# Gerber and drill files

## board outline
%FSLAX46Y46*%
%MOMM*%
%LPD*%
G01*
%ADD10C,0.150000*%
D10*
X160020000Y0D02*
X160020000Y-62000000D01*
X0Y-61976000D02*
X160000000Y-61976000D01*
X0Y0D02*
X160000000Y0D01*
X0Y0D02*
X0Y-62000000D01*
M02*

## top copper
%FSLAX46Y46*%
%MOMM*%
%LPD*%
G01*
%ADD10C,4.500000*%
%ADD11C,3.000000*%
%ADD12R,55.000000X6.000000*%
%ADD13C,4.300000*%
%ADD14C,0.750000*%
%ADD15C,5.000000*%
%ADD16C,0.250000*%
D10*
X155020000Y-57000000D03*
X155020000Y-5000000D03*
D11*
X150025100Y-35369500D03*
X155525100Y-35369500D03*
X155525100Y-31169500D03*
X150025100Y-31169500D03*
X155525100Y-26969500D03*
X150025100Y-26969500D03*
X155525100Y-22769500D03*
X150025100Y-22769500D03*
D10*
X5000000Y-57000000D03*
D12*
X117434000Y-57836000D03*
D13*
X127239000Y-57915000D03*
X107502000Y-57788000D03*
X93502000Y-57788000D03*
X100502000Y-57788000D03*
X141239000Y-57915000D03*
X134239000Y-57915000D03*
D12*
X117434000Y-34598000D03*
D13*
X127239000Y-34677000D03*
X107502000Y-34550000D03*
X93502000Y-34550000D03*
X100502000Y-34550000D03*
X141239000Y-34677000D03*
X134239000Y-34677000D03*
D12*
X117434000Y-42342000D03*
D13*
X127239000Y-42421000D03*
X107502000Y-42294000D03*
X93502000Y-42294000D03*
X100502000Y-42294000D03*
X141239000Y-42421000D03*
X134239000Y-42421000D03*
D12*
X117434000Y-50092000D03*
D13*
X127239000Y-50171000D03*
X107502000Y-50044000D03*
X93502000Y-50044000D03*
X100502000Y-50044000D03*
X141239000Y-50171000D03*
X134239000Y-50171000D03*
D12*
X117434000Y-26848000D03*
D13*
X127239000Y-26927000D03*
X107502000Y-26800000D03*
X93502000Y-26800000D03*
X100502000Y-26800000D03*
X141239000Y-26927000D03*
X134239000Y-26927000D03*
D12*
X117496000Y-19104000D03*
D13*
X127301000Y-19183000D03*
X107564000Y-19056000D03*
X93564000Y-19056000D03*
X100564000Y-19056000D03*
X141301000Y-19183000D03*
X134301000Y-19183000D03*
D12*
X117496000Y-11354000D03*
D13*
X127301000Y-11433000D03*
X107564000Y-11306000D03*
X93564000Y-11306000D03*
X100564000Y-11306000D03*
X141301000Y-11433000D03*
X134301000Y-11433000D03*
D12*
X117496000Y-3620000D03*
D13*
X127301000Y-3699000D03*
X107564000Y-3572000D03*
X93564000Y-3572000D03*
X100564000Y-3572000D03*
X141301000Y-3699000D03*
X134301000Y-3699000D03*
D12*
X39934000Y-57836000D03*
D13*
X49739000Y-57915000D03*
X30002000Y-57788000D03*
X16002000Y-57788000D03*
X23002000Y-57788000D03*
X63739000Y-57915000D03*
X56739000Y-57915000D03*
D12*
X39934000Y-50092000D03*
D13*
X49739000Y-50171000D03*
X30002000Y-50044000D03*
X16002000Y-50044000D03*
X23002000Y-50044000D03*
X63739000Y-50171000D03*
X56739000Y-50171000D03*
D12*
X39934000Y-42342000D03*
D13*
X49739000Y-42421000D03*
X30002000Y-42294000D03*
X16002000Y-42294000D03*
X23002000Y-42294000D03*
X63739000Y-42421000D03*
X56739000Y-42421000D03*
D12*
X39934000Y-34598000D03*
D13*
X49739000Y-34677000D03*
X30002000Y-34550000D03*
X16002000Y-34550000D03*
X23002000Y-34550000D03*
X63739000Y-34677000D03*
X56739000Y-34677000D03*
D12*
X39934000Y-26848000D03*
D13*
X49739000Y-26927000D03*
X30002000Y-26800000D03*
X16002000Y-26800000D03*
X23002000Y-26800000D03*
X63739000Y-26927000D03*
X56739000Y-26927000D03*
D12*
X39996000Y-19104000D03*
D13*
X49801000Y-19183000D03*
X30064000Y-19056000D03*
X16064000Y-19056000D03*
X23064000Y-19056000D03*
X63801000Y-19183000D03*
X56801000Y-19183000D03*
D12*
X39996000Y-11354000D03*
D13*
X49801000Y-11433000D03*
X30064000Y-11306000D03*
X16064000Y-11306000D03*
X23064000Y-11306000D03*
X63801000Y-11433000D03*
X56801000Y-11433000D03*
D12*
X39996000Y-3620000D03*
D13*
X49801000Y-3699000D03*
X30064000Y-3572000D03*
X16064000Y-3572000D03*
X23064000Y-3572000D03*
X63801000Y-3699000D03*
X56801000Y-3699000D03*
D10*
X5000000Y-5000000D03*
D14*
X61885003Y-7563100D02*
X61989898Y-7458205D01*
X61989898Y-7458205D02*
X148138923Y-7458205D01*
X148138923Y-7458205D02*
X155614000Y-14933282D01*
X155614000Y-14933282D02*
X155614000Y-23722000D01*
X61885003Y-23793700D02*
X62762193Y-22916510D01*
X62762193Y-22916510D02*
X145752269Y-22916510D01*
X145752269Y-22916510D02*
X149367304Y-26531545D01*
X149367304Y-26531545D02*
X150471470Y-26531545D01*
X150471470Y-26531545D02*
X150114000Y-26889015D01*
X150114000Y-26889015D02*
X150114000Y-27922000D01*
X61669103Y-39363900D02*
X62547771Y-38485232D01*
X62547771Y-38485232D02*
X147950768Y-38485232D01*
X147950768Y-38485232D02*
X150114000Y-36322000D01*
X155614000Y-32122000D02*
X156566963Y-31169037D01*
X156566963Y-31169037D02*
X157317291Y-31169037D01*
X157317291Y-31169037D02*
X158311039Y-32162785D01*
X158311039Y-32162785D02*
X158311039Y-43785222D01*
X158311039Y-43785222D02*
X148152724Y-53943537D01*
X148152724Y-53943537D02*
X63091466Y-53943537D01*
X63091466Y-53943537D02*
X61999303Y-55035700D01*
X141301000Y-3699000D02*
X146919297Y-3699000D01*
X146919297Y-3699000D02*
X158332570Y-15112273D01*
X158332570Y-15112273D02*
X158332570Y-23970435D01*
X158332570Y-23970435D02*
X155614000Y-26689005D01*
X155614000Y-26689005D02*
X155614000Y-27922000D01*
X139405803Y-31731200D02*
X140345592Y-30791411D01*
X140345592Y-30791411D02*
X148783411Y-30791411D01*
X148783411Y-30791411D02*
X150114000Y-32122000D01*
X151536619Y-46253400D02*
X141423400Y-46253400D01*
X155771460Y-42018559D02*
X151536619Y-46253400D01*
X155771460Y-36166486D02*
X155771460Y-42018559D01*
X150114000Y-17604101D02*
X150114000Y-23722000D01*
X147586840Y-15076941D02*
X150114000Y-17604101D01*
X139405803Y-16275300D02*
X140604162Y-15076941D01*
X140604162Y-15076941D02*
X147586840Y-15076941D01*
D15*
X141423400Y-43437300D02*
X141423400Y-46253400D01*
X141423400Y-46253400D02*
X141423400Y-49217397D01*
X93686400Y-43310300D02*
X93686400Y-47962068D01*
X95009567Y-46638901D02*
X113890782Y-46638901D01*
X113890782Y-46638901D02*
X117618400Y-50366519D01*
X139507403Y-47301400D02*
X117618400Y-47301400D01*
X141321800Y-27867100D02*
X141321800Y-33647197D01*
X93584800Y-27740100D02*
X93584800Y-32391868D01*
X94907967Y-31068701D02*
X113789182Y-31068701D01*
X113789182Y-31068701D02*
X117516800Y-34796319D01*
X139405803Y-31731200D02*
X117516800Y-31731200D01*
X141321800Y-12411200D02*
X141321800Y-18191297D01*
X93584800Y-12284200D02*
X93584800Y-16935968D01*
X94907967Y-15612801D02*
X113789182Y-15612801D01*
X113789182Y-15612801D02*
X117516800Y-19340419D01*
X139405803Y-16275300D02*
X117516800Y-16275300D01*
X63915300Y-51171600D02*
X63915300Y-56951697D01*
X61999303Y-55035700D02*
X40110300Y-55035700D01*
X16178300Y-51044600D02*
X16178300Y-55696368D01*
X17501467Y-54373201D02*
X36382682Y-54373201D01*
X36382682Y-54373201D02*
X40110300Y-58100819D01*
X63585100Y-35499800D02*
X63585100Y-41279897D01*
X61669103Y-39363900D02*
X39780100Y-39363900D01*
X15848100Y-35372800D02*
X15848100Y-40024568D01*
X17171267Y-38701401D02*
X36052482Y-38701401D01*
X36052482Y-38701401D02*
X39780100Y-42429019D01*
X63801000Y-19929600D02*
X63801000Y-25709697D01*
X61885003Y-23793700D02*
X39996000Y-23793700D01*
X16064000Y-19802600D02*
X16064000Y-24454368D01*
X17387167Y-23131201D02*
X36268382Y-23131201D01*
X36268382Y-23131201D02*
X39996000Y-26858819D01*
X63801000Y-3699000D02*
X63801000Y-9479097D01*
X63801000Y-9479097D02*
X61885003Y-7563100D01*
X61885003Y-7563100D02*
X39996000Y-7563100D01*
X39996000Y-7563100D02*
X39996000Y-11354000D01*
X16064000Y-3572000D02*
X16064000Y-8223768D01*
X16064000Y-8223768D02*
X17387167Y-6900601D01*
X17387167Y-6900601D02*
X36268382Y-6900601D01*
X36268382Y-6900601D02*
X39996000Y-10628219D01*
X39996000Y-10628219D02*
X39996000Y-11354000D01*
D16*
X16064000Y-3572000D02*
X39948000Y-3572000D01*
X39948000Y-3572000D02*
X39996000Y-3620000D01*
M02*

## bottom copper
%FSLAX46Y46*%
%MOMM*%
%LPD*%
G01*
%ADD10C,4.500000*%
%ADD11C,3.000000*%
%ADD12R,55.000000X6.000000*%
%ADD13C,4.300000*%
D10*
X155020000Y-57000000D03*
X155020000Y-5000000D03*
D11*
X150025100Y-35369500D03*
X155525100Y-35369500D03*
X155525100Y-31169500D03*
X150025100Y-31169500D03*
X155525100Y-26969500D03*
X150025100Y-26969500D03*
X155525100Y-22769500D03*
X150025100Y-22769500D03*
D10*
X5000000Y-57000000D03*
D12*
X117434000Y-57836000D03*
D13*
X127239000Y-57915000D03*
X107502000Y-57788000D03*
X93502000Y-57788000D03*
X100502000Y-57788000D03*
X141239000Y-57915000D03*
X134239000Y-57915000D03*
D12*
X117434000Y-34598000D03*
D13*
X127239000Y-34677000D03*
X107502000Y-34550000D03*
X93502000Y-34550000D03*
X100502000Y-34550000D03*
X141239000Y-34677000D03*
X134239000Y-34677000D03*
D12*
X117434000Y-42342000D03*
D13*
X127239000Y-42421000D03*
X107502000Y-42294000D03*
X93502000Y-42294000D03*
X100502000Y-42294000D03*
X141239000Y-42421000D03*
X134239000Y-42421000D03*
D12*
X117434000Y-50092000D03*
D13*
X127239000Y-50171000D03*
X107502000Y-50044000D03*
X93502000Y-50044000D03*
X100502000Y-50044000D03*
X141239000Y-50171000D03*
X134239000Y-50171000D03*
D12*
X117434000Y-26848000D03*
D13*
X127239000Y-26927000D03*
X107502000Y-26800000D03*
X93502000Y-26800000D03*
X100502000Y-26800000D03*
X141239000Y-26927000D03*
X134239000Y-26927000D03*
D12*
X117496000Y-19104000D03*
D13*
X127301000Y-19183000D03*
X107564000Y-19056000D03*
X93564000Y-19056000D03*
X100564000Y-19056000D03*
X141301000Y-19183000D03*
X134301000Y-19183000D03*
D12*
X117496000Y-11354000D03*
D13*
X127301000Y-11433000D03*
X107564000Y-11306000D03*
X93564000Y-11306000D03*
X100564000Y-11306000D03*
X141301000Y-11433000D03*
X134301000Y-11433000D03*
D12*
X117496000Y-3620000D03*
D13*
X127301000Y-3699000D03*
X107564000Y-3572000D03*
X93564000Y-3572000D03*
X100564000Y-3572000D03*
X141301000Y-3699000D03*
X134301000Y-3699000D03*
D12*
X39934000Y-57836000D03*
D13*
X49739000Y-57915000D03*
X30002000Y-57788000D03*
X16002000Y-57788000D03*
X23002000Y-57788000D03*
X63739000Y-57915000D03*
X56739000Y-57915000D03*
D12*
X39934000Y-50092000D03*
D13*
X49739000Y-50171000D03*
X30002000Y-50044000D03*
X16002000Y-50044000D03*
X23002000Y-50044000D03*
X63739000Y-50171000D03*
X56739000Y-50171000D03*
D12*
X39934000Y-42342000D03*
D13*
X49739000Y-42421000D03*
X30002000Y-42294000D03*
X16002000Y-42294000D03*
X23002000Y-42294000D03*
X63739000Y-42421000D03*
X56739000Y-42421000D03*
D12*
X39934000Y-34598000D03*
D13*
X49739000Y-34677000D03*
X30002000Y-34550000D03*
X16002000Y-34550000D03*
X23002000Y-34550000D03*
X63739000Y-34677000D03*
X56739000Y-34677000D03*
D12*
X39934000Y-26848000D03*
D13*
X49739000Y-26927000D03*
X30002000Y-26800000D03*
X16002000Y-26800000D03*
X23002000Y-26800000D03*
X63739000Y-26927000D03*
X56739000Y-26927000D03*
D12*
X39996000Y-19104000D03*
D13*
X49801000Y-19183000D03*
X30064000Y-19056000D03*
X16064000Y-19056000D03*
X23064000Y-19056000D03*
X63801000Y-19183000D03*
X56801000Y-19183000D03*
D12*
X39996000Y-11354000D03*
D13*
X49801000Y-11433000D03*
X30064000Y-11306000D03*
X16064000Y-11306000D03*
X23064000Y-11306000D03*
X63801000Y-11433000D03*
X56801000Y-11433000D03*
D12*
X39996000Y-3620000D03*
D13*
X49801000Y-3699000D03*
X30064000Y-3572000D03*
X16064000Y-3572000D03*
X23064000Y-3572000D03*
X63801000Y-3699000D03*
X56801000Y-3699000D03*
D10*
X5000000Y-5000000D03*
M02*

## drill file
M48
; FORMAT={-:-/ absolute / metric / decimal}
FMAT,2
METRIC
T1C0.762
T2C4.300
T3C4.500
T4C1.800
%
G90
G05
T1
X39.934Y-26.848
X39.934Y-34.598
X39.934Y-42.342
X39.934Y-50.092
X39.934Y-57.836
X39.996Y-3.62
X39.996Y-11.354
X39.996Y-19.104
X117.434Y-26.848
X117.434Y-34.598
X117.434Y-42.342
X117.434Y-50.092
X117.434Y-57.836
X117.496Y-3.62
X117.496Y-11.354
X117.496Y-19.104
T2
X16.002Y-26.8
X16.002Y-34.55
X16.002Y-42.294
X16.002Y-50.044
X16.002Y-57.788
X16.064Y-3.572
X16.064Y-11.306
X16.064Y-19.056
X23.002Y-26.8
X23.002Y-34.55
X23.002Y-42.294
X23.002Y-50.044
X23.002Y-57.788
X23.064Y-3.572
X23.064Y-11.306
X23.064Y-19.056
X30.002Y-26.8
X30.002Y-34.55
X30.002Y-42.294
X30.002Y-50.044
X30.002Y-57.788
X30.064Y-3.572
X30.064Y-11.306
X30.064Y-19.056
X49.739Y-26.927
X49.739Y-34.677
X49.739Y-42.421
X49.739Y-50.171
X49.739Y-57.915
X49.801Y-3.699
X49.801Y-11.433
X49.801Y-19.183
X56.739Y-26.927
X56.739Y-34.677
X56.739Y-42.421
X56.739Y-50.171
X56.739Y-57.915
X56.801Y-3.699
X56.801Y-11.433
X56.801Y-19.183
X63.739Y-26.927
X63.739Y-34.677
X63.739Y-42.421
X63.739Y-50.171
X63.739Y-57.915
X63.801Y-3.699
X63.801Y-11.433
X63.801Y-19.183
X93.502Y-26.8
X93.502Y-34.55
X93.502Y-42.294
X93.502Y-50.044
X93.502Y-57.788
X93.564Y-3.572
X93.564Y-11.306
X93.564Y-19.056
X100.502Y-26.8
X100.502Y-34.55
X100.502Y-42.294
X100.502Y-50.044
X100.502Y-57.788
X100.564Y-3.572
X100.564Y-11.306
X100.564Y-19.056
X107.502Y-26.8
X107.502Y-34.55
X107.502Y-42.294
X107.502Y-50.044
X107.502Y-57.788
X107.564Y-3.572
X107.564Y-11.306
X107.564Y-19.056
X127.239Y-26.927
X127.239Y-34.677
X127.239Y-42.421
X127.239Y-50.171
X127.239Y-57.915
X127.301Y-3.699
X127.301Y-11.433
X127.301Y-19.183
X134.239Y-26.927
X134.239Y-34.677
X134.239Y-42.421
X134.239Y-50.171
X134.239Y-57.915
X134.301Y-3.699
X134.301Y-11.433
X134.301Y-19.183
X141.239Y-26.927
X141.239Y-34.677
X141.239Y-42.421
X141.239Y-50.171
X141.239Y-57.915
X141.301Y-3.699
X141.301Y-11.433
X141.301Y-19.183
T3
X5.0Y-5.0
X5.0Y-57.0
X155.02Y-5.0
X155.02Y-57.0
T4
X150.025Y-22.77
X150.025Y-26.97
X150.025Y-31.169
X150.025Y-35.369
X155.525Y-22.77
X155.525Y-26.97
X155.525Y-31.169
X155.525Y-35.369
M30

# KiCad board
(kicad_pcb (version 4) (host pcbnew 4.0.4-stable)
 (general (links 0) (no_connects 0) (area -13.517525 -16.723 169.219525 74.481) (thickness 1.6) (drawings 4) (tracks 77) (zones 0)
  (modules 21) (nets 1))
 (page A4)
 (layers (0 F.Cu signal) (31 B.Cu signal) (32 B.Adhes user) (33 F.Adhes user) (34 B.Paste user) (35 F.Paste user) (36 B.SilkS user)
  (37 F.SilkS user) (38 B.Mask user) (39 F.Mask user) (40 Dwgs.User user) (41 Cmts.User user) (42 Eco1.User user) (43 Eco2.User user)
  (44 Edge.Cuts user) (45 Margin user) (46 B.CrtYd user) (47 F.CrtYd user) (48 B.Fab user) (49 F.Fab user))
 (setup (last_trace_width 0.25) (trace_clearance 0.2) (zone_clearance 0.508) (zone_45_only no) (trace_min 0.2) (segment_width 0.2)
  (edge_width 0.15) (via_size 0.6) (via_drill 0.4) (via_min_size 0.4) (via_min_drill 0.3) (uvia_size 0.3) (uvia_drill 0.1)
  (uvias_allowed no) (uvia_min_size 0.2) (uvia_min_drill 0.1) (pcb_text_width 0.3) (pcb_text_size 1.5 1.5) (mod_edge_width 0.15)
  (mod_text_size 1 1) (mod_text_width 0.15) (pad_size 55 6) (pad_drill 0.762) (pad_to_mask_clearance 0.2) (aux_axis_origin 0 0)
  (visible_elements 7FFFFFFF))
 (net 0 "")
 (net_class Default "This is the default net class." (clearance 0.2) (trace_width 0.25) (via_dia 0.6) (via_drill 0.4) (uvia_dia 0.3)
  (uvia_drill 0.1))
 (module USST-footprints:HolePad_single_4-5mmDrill (layer F.Cu) (at 154.258 49.634)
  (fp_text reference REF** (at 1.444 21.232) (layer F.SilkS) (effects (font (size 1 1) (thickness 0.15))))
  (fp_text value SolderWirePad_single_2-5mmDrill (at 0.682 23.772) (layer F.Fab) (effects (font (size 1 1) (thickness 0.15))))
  (pad "" thru_hole circle (at 0.762 7.366) (size 4.5 4.5) (drill 4.5) (layers *.Cu *.Mask)))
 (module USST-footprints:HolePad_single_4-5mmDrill (layer F.Cu) (at 154.258 -2.366)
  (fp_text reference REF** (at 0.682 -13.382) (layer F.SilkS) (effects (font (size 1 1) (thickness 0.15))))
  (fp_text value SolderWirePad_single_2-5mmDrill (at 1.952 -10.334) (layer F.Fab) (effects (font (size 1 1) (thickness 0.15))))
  (pad "" thru_hole circle (at 0.762 7.366) (size 4.5 4.5) (drill 4.5) (layers *.Cu *.Mask)))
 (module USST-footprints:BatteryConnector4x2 (layer F.Cu) (at 150.0251 35.3695)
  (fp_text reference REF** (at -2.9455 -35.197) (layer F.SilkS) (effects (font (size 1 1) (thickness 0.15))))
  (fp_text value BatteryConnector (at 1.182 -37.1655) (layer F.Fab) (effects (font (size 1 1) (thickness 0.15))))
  (pad "" np_thru_hole circle (at 0 0) (size 3 3) (drill 1.8) (layers *.Cu))
  (pad "" np_thru_hole circle (at 5.5 0) (size 3 3) (drill 1.8) (layers *.Cu))
  (pad "" np_thru_hole circle (at 5.5 -4.2) (size 3 3) (drill 1.8) (layers *.Cu))
  (pad "" np_thru_hole circle (at 0 -4.2) (size 3 3) (drill 1.8) (layers *.Cu))
  (pad "" np_thru_hole circle (at 5.5 -8.4) (size 3 3) (drill 1.8) (layers *.Cu))
  (pad "" np_thru_hole circle (at 0 -8.4) (size 3 3) (drill 1.8) (layers *.Cu))
  (pad "" np_thru_hole circle (at 5.5 -12.6) (size 3 3) (drill 1.8) (layers *.Cu))
  (pad "" np_thru_hole circle (at 0 -12.6) (size 3 3) (drill 1.8) (layers *.Cu)))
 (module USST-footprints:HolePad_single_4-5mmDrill (layer F.Cu) (at 4.238 49.634)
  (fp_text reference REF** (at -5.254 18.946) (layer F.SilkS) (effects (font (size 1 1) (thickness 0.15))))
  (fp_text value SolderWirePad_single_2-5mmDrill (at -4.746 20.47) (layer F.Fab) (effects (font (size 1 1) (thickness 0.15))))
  (pad "" thru_hole circle (at 0.762 7.366) (size 4.5 4.5) (drill 4.5) (layers *.Cu *.Mask)))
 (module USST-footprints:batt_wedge (layer F.Cu) (at 117.434 57.836)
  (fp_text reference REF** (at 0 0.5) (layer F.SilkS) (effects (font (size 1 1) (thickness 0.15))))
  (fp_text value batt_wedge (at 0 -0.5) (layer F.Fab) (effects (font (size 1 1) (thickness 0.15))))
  (pad 8 thru_hole rect (at 0 0) (size 55 6) (drill 0.762) (layers F.Cu F.Paste))
  (pad "" thru_hole circle (at 9.805 0.079) (size 4.3 4.3) (drill 4.3) (layers *.Cu *.Mask))
  (pad "" thru_hole circle (at -9.932 -0.048) (size 4.3 4.3) (drill 4.3) (layers *.Cu *.Mask))
  (pad "" thru_hole circle (at -23.932 -0.048) (size 4.3 4.3) (drill 4.3) (layers *.Cu *.Mask))
  (pad "" thru_hole circle (at -16.932 -0.048) (size 4.3 4.3) (drill 4.3) (layers *.Cu *.Mask))
  (pad "" thru_hole circle (at 23.805 0.079) (size 4.3 4.3) (drill 4.3) (layers *.Cu *.Mask))
  (pad "" thru_hole circle (at 16.805 0.079) (size 4.3 4.3) (drill 4.3) (layers *.Cu *.Mask)))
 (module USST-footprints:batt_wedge (layer F.Cu) (at 117.434 34.598)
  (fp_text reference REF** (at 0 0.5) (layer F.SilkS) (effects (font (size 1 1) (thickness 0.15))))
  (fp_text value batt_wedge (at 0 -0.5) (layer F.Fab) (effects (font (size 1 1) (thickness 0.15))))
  (pad 5 thru_hole rect (at 0 0) (size 55 6) (drill 0.762) (layers F.Cu F.Paste))
  (pad "" thru_hole circle (at 9.805 0.079) (size 4.3 4.3) (drill 4.3) (layers *.Cu *.Mask))
  (pad "" thru_hole circle (at -9.932 -0.048) (size 4.3 4.3) (drill 4.3) (layers *.Cu *.Mask))
  (pad "" thru_hole circle (at -23.932 -0.048) (size 4.3 4.3) (drill 4.3) (layers *.Cu *.Mask))
  (pad "" thru_hole circle (at -16.932 -0.048) (size 4.3 4.3) (drill 4.3) (layers *.Cu *.Mask))
  (pad "" thru_hole circle (at 23.805 0.079) (size 4.3 4.3) (drill 4.3) (layers *.Cu *.Mask))
  (pad "" thru_hole circle (at 16.805 0.079) (size 4.3 4.3) (drill 4.3) (layers *.Cu *.Mask)))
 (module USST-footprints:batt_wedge (layer F.Cu) (at 117.434 42.342)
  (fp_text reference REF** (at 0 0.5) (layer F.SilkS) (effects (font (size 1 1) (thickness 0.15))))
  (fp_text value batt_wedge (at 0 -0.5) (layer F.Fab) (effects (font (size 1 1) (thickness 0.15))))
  (pad 6 thru_hole rect (at 0 0) (size 55 6) (drill 0.762) (layers F.Cu F.Paste))
  (pad "" thru_hole circle (at 9.805 0.079) (size 4.3 4.3) (drill 4.3) (layers *.Cu *.Mask))
  (pad "" thru_hole circle (at -9.932 -0.048) (size 4.3 4.3) (drill 4.3) (layers *.Cu *.Mask))
  (pad "" thru_hole circle (at -23.932 -0.048) (size 4.3 4.3) (drill 4.3) (layers *.Cu *.Mask))
  (pad "" thru_hole circle (at -16.932 -0.048) (size 4.3 4.3) (drill 4.3) (layers *.Cu *.Mask))
  (pad "" thru_hole circle (at 23.805 0.079) (size 4.3 4.3) (drill 4.3) (layers *.Cu *.Mask))
  (pad "" thru_hole circle (at 16.805 0.079) (size 4.3 4.3) (drill 4.3) (layers *.Cu *.Mask)))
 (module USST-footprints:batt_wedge (layer F.Cu) (at 117.434 50.092)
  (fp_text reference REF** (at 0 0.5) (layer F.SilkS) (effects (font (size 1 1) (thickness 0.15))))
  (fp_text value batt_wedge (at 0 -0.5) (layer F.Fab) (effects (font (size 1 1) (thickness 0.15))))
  (pad 7 thru_hole rect (at 0 0) (size 55 6) (drill 0.762) (layers F.Cu F.Paste))
  (pad "" thru_hole circle (at 9.805 0.079) (size 4.3 4.3) (drill 4.3) (layers *.Cu *.Mask))
  (pad "" thru_hole circle (at -9.932 -0.048) (size 4.3 4.3) (drill 4.3) (layers *.Cu *.Mask))
  (pad "" thru_hole circle (at -23.932 -0.048) (size 4.3 4.3) (drill 4.3) (layers *.Cu *.Mask))
  (pad "" thru_hole circle (at -16.932 -0.048) (size 4.3 4.3) (drill 4.3) (layers *.Cu *.Mask))
  (pad "" thru_hole circle (at 23.805 0.079) (size 4.3 4.3) (drill 4.3) (layers *.Cu *.Mask))
  (pad "" thru_hole circle (at 16.805 0.079) (size 4.3 4.3) (drill 4.3) (layers *.Cu *.Mask)))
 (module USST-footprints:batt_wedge (layer F.Cu) (at 117.434 26.848)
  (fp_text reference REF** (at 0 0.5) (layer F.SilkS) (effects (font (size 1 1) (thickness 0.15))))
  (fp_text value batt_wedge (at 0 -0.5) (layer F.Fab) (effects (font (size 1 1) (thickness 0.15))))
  (pad 4 thru_hole rect (at 0 0) (size 55 6) (drill 0.762) (layers F.Cu F.Paste))
  (pad "" thru_hole circle (at 9.805 0.079) (size 4.3 4.3) (drill 4.3) (layers *.Cu *.Mask))
  (pad "" thru_hole circle (at -9.932 -0.048) (size 4.3 4.3) (drill 4.3) (layers *.Cu *.Mask))
  (pad "" thru_hole circle (at -23.932 -0.048) (size 4.3 4.3) (drill 4.3) (layers *.Cu *.Mask))
  (pad "" thru_hole circle (at -16.932 -0.048) (size 4.3 4.3) (drill 4.3) (layers *.Cu *.Mask))
  (pad "" thru_hole circle (at 23.805 0.079) (size 4.3 4.3) (drill 4.3) (layers *.Cu *.Mask))
  (pad "" thru_hole circle (at 16.805 0.079) (size 4.3 4.3) (drill 4.3) (layers *.Cu *.Mask)))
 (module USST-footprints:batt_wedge (layer F.Cu) (at 117.496 19.104)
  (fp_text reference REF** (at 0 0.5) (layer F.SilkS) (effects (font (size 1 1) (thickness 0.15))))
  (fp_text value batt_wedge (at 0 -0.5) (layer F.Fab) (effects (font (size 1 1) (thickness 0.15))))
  (pad 3 thru_hole rect (at 0 0) (size 55 6) (drill 0.762) (layers F.Cu F.Paste))
  (pad "" thru_hole circle (at 9.805 0.079) (size 4.3 4.3) (drill 4.3) (layers *.Cu *.Mask))
  (pad "" thru_hole circle (at -9.932 -0.048) (size 4.3 4.3) (drill 4.3) (layers *.Cu *.Mask))
  (pad "" thru_hole circle (at -23.932 -0.048) (size 4.3 4.3) (drill 4.3) (layers *.Cu *.Mask))
  (pad "" thru_hole circle (at -16.932 -0.048) (size 4.3 4.3) (drill 4.3) (layers *.Cu *.Mask))
  (pad "" thru_hole circle (at 23.805 0.079) (size 4.3 4.3) (drill 4.3) (layers *.Cu *.Mask))
  (pad "" thru_hole circle (at 16.805 0.079) (size 4.3 4.3) (drill 4.3) (layers *.Cu *.Mask)))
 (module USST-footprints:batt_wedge (layer F.Cu) (at 117.496 11.354)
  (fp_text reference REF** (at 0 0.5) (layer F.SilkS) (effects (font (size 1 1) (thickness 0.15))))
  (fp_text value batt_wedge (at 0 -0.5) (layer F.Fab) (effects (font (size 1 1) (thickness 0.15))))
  (pad 2 thru_hole rect (at 0 0) (size 55 6) (drill 0.762) (layers F.Cu F.Paste))
  (pad "" thru_hole circle (at 9.805 0.079) (size 4.3 4.3) (drill 4.3) (layers *.Cu *.Mask))
  (pad "" thru_hole circle (at -9.932 -0.048) (size 4.3 4.3) (drill 4.3) (layers *.Cu *.Mask))
  (pad "" thru_hole circle (at -23.932 -0.048) (size 4.3 4.3) (drill 4.3) (layers *.Cu *.Mask))
  (pad "" thru_hole circle (at -16.932 -0.048) (size 4.3 4.3) (drill 4.3) (layers *.Cu *.Mask))
  (pad "" thru_hole circle (at 23.805 0.079) (size 4.3 4.3) (drill 4.3) (layers *.Cu *.Mask))
  (pad "" thru_hole circle (at 16.805 0.079) (size 4.3 4.3) (drill 4.3) (layers *.Cu *.Mask)))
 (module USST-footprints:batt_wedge (layer F.Cu) (at 117.496 3.62)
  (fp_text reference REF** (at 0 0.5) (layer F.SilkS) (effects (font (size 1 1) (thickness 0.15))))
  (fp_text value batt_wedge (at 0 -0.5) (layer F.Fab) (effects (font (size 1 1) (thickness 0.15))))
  (pad 1 thru_hole rect (at 0 0) (size 55 6) (drill 0.762) (layers F.Cu F.Paste))
  (pad "" thru_hole circle (at 9.805 0.079) (size 4.3 4.3) (drill 4.3) (layers *.Cu *.Mask))
  (pad "" thru_hole circle (at -9.932 -0.048) (size 4.3 4.3) (drill 4.3) (layers *.Cu *.Mask))
  (pad "" thru_hole circle (at -23.932 -0.048) (size 4.3 4.3) (drill 4.3) (layers *.Cu *.Mask))
  (pad "" thru_hole circle (at -16.932 -0.048) (size 4.3 4.3) (drill 4.3) (layers *.Cu *.Mask))
  (pad "" thru_hole circle (at 23.805 0.079) (size 4.3 4.3) (drill 4.3) (layers *.Cu *.Mask))
  (pad "" thru_hole circle (at 16.805 0.079) (size 4.3 4.3) (drill 4.3) (layers *.Cu *.Mask)))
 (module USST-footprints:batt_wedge (layer F.Cu) (at 39.934 57.836)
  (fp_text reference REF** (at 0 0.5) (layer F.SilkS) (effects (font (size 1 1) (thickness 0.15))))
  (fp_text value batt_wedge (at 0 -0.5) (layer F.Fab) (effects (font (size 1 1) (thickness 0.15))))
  (pad 8 thru_hole rect (at 0 0) (size 55 6) (drill 0.762) (layers F.Cu F.Paste))
  (pad "" thru_hole circle (at 9.805 0.079) (size 4.3 4.3) (drill 4.3) (layers *.Cu *.Mask))
  (pad "" thru_hole circle (at -9.932 -0.048) (size 4.3 4.3) (drill 4.3) (layers *.Cu *.Mask))
  (pad "" thru_hole circle (at -23.932 -0.048) (size 4.3 4.3) (drill 4.3) (layers *.Cu *.Mask))
  (pad "" thru_hole circle (at -16.932 -0.048) (size 4.3 4.3) (drill 4.3) (layers *.Cu *.Mask))
  (pad "" thru_hole circle (at 23.805 0.079) (size 4.3 4.3) (drill 4.3) (layers *.Cu *.Mask))
  (pad "" thru_hole circle (at 16.805 0.079) (size 4.3 4.3) (drill 4.3) (layers *.Cu *.Mask)))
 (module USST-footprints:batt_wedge (layer F.Cu) (at 39.934 50.092)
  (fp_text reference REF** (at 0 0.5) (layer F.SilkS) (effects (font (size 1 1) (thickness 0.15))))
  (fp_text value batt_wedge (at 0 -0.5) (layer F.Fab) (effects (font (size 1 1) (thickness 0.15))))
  (pad 7 thru_hole rect (at 0 0) (size 55 6) (drill 0.762) (layers F.Cu F.Paste))
  (pad "" thru_hole circle (at 9.805 0.079) (size 4.3 4.3) (drill 4.3) (layers *.Cu *.Mask))
  (pad "" thru_hole circle (at -9.932 -0.048) (size 4.3 4.3) (drill 4.3) (layers *.Cu *.Mask))
  (pad "" thru_hole circle (at -23.932 -0.048) (size 4.3 4.3) (drill 4.3) (layers *.Cu *.Mask))
  (pad "" thru_hole circle (at -16.932 -0.048) (size 4.3 4.3) (drill 4.3) (layers *.Cu *.Mask))
  (pad "" thru_hole circle (at 23.805 0.079) (size 4.3 4.3) (drill 4.3) (layers *.Cu *.Mask))
  (pad "" thru_hole circle (at 16.805 0.079) (size 4.3 4.3) (drill 4.3) (layers *.Cu *.Mask)))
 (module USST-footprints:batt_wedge (layer F.Cu) (at 39.934 42.342)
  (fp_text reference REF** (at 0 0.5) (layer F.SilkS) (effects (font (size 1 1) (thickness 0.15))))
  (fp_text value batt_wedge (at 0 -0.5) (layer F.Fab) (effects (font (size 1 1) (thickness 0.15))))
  (pad 6 thru_hole rect (at 0 0) (size 55 6) (drill 0.762) (layers F.Cu F.Paste))
  (pad "" thru_hole circle (at 9.805 0.079) (size 4.3 4.3) (drill 4.3) (layers *.Cu *.Mask))
  (pad "" thru_hole circle (at -9.932 -0.048) (size 4.3 4.3) (drill 4.3) (layers *.Cu *.Mask))
  (pad "" thru_hole circle (at -23.932 -0.048) (size 4.3 4.3) (drill 4.3) (layers *.Cu *.Mask))
  (pad "" thru_hole circle (at -16.932 -0.048) (size 4.3 4.3) (drill 4.3) (layers *.Cu *.Mask))
  (pad "" thru_hole circle (at 23.805 0.079) (size 4.3 4.3) (drill 4.3) (layers *.Cu *.Mask))
  (pad "" thru_hole circle (at 16.805 0.079) (size 4.3 4.3) (drill 4.3) (layers *.Cu *.Mask)))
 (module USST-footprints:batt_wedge (layer F.Cu) (at 39.934 34.598)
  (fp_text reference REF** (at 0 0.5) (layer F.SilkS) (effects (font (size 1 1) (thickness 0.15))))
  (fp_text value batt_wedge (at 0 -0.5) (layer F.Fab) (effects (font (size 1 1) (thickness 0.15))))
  (pad 5 thru_hole rect (at 0 0) (size 55 6) (drill 0.762) (layers F.Cu F.Paste))
  (pad "" thru_hole circle (at 9.805 0.079) (size 4.3 4.3) (drill 4.3) (layers *.Cu *.Mask))
  (pad "" thru_hole circle (at -9.932 -0.048) (size 4.3 4.3) (drill 4.3) (layers *.Cu *.Mask))
  (pad "" thru_hole circle (at -23.932 -0.048) (size 4.3 4.3) (drill 4.3) (layers *.Cu *.Mask))
  (pad "" thru_hole circle (at -16.932 -0.048) (size 4.3 4.3) (drill 4.3) (layers *.Cu *.Mask))
  (pad "" thru_hole circle (at 23.805 0.079) (size 4.3 4.3) (drill 4.3) (layers *.Cu *.Mask))
  (pad "" thru_hole circle (at 16.805 0.079) (size 4.3 4.3) (drill 4.3) (layers *.Cu *.Mask)))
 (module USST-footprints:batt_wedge (layer F.Cu) (at 39.934 26.848)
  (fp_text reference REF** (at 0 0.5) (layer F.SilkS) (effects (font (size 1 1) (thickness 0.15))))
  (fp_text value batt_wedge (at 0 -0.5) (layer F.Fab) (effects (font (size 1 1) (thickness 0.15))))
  (pad 4 thru_hole rect (at 0 0) (size 55 6) (drill 0.762) (layers F.Cu F.Paste))
  (pad "" thru_hole circle (at 9.805 0.079) (size 4.3 4.3) (drill 4.3) (layers *.Cu *.Mask))
  (pad "" thru_hole circle (at -9.932 -0.048) (size 4.3 4.3) (drill 4.3) (layers *.Cu *.Mask))
  (pad "" thru_hole circle (at -23.932 -0.048) (size 4.3 4.3) (drill 4.3) (layers *.Cu *.Mask))
  (pad "" thru_hole circle (at -16.932 -0.048) (size 4.3 4.3) (drill 4.3) (layers *.Cu *.Mask))
  (pad "" thru_hole circle (at 23.805 0.079) (size 4.3 4.3) (drill 4.3) (layers *.Cu *.Mask))
  (pad "" thru_hole circle (at 16.805 0.079) (size 4.3 4.3) (drill 4.3) (layers *.Cu *.Mask)))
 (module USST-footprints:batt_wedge (layer F.Cu) (at 39.996 19.104)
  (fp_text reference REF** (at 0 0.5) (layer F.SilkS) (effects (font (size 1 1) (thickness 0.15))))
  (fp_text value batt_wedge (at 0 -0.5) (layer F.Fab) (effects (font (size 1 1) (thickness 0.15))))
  (pad 3 thru_hole rect (at 0 0) (size 55 6) (drill 0.762) (layers F.Cu F.Paste))
  (pad "" thru_hole circle (at 9.805 0.079) (size 4.3 4.3) (drill 4.3) (layers *.Cu *.Mask))
  (pad "" thru_hole circle (at -9.932 -0.048) (size 4.3 4.3) (drill 4.3) (layers *.Cu *.Mask))
  (pad "" thru_hole circle (at -23.932 -0.048) (size 4.3 4.3) (drill 4.3) (layers *.Cu *.Mask))
  (pad "" thru_hole circle (at -16.932 -0.048) (size 4.3 4.3) (drill 4.3) (layers *.Cu *.Mask))
  (pad "" thru_hole circle (at 23.805 0.079) (size 4.3 4.3) (drill 4.3) (layers *.Cu *.Mask))
  (pad "" thru_hole circle (at 16.805 0.079) (size 4.3 4.3) (drill 4.3) (layers *.Cu *.Mask)))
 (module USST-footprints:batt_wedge (layer F.Cu) (at 39.996 11.354)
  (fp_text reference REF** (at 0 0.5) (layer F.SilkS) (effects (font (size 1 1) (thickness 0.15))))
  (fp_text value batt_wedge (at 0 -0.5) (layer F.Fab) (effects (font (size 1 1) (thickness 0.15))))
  (pad 2 thru_hole rect (at 0 0) (size 55 6) (drill 0.762) (layers F.Cu F.Paste))
  (pad "" thru_hole circle (at 9.805 0.079) (size 4.3 4.3) (drill 4.3) (layers *.Cu *.Mask))
  (pad "" thru_hole circle (at -9.932 -0.048) (size 4.3 4.3) (drill 4.3) (layers *.Cu *.Mask))
  (pad "" thru_hole circle (at -23.932 -0.048) (size 4.3 4.3) (drill 4.3) (layers *.Cu *.Mask))
  (pad "" thru_hole circle (at -16.932 -0.048) (size 4.3 4.3) (drill 4.3) (layers *.Cu *.Mask))
  (pad "" thru_hole circle (at 23.805 0.079) (size 4.3 4.3) (drill 4.3) (layers *.Cu *.Mask))
  (pad "" thru_hole circle (at 16.805 0.079) (size 4.3 4.3) (drill 4.3) (layers *.Cu *.Mask)))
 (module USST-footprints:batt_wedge (layer F.Cu) (at 39.996 3.62)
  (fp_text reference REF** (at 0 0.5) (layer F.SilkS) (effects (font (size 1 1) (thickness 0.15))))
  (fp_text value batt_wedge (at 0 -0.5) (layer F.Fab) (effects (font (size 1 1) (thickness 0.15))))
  (pad 1 thru_hole rect (at 0 0) (size 55 6) (drill 0.762) (layers F.Cu F.Paste))
  (pad "" thru_hole circle (at 9.805 0.079) (size 4.3 4.3) (drill 4.3) (layers *.Cu *.Mask))
  (pad "" thru_hole circle (at -9.932 -0.048) (size 4.3 4.3) (drill 4.3) (layers *.Cu *.Mask))
  (pad "" thru_hole circle (at -23.932 -0.048) (size 4.3 4.3) (drill 4.3) (layers *.Cu *.Mask))
  (pad "" thru_hole circle (at -16.932 -0.048) (size 4.3 4.3) (drill 4.3) (layers *.Cu *.Mask))
  (pad "" thru_hole circle (at 23.805 0.079) (size 4.3 4.3) (drill 4.3) (layers *.Cu *.Mask))
  (pad "" thru_hole circle (at 16.805 0.079) (size 4.3 4.3) (drill 4.3) (layers *.Cu *.Mask)))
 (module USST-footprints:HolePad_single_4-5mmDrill (layer F.Cu) (at 4.238 -2.366)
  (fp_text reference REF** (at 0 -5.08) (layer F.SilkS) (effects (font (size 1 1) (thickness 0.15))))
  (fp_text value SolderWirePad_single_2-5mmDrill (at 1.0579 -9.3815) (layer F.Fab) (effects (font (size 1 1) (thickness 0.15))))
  (pad "" thru_hole circle (at 0.762 7.366) (size 4.5 4.5) (drill 4.5) (layers *.Cu *.Mask)))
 (gr_line (start 160.02 0) (end 160.02 62) (layer Edge.Cuts) (width 0.15))
 (gr_line (start 0 61.976) (end 160 61.976) (layer Edge.Cuts) (width 0.15))
 (gr_line (start 0 0) (end 160 0) (layer Edge.Cuts) (width 0.15))
 (gr_line (start 0 0) (end 0 62) (layer Edge.Cuts) (width 0.15))
 (segment (start 61.885003 7.5631) (end 61.989898 7.458205) (width 0.75) (layer F.Cu) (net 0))
 (segment (start 61.989898 7.458205) (end 148.138923 7.458205) (width 0.75) (layer F.Cu) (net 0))
 (segment (start 148.138923 7.458205) (end 155.614 14.933282) (width 0.75) (layer F.Cu) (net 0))
 (segment (start 155.614 14.933282) (end 155.614 23.722) (width 0.75) (layer F.Cu) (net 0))
 (segment (start 61.885003 23.7937) (end 62.762193 22.91651) (width 0.75) (layer F.Cu) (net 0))
 (segment (start 62.762193 22.91651) (end 145.752269 22.91651) (width 0.75) (layer F.Cu) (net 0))
 (segment (start 145.752269 22.91651) (end 149.367304 26.531545) (width 0.75) (layer F.Cu) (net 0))
 (segment (start 149.367304 26.531545) (end 150.47147 26.531545) (width 0.75) (layer F.Cu) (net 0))
 (segment (start 150.47147 26.531545) (end 150.114 26.889015) (width 0.75) (layer F.Cu) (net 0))
 (segment (start 150.114 26.889015) (end 150.114 27.922) (width 0.75) (layer F.Cu) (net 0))
 (segment (start 61.669103 39.3639) (end 62.547771 38.485232) (width 0.75) (layer F.Cu) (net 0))
 (segment (start 62.547771 38.485232) (end 147.950768 38.485232) (width 0.75) (layer F.Cu) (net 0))
 (segment (start 147.950768 38.485232) (end 150.114 36.322) (width 0.75) (layer F.Cu) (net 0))
 (segment (start 155.614 32.122) (end 156.566963 31.169037) (width 0.75) (layer F.Cu) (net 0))
 (segment (start 156.566963 31.169037) (end 157.317291 31.169037) (width 0.75) (layer F.Cu) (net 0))
 (segment (start 157.317291 31.169037) (end 158.311039 32.162785) (width 0.75) (layer F.Cu) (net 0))
 (segment (start 158.311039 32.162785) (end 158.311039 43.785222) (width 0.75) (layer F.Cu) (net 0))
 (segment (start 158.311039 43.785222) (end 148.152724 53.943537) (width 0.75) (layer F.Cu) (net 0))
 (segment (start 148.152724 53.943537) (end 63.091466 53.943537) (width 0.75) (layer F.Cu) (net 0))
 (segment (start 63.091466 53.943537) (end 61.999303 55.0357) (width 0.75) (layer F.Cu) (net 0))
 (segment (start 141.301 3.699) (end 146.919297 3.699) (width 0.75) (layer F.Cu) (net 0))
 (segment (start 146.919297 3.699) (end 158.33257 15.112273) (width 0.75) (layer F.Cu) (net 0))
 (segment (start 158.33257 15.112273) (end 158.33257 23.970435) (width 0.75) (layer F.Cu) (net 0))
 (segment (start 158.33257 23.970435) (end 155.614 26.689005) (width 0.75) (layer F.Cu) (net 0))
 (segment (start 155.614 26.689005) (end 155.614 27.922) (width 0.75) (layer F.Cu) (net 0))
 (segment (start 139.405803 31.7312) (end 140.345592 30.791411) (width 0.75) (layer F.Cu) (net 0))
 (segment (start 140.345592 30.791411) (end 148.783411 30.791411) (width 0.75) (layer F.Cu) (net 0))
 (segment (start 148.783411 30.791411) (end 150.114 32.122) (width 0.75) (layer F.Cu) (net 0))
 (segment (start 151.536619 46.2534) (end 141.4234 46.2534) (width 0.75) (layer F.Cu) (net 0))
 (segment (start 155.77146 42.018559) (end 151.536619 46.2534) (width 0.75) (layer F.Cu) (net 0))
 (segment (start 155.77146 36.166486) (end 155.77146 42.018559) (width 0.75) (layer F.Cu) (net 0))
 (segment (start 150.114 17.604101) (end 150.114 23.722) (width 0.75) (layer F.Cu) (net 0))
 (segment (start 147.58684 15.076941) (end 150.114 17.604101) (width 0.75) (layer F.Cu) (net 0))
 (segment (start 139.405803 16.2753) (end 140.604162 15.076941) (width 0.75) (layer F.Cu) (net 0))
 (segment (start 140.604162 15.076941) (end 147.58684 15.076941) (width 0.75) (layer F.Cu) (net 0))
 (segment (start 141.4234 43.4373) (end 141.4234 46.2534) (width 5) (layer F.Cu) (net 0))
 (segment (start 141.4234 46.2534) (end 141.4234 49.217397) (width 5) (layer F.Cu) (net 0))
 (segment (start 93.6864 43.3103) (end 93.6864 47.962068) (width 5) (layer F.Cu) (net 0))
 (segment (start 95.009567 46.638901) (end 113.890782 46.638901) (width 5) (layer F.Cu) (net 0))
 (segment (start 113.890782 46.638901) (end 117.6184 50.366519) (width 5) (layer F.Cu) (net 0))
 (segment (start 139.507403 47.3014) (end 117.6184 47.3014) (width 5) (layer F.Cu) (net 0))
 (segment (start 141.3218 27.8671) (end 141.3218 33.647197) (width 5) (layer F.Cu) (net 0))
 (segment (start 93.5848 27.7401) (end 93.5848 32.391868) (width 5) (layer F.Cu) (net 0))
 (segment (start 94.907967 31.068701) (end 113.789182 31.068701) (width 5) (layer F.Cu) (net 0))
 (segment (start 113.789182 31.068701) (end 117.5168 34.796319) (width 5) (layer F.Cu) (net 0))
 (segment (start 139.405803 31.7312) (end 117.5168 31.7312) (width 5) (layer F.Cu) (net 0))
 (segment (start 141.3218 12.4112) (end 141.3218 18.191297) (width 5) (layer F.Cu) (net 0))
 (segment (start 93.5848 12.2842) (end 93.5848 16.935968) (width 5) (layer F.Cu) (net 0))
 (segment (start 94.907967 15.612801) (end 113.789182 15.612801) (width 5) (layer F.Cu) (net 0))
 (segment (start 113.789182 15.612801) (end 117.5168 19.340419) (width 5) (layer F.Cu) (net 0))
 (segment (start 139.405803 16.2753) (end 117.5168 16.2753) (width 5) (layer F.Cu) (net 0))
 (segment (start 63.9153 51.1716) (end 63.9153 56.951697) (width 5) (layer F.Cu) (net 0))
 (segment (start 61.999303 55.0357) (end 40.1103 55.0357) (width 5) (layer F.Cu) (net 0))
 (segment (start 16.1783 51.0446) (end 16.1783 55.696368) (width 5) (layer F.Cu) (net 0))
 (segment (start 17.501467 54.373201) (end 36.382682 54.373201) (width 5) (layer F.Cu) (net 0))
 (segment (start 36.382682 54.373201) (end 40.1103 58.100819) (width 5) (layer F.Cu) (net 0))
 (segment (start 63.5851 35.4998) (end 63.5851 41.279897) (width 5) (layer F.Cu) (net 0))
 (segment (start 61.669103 39.3639) (end 39.7801 39.3639) (width 5) (layer F.Cu) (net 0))
 (segment (start 15.8481 35.3728) (end 15.8481 40.024568) (width 5) (layer F.Cu) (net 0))
 (segment (start 17.171267 38.701401) (end 36.052482 38.701401) (width 5) (layer F.Cu) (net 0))
 (segment (start 36.052482 38.701401) (end 39.7801 42.429019) (width 5) (layer F.Cu) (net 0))
 (segment (start 63.801 19.9296) (end 63.801 25.709697) (width 5) (layer F.Cu) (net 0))
 (segment (start 61.885003 23.7937) (end 39.996 23.7937) (width 5) (layer F.Cu) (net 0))
 (segment (start 16.064 19.8026) (end 16.064 24.454368) (width 5) (layer F.Cu) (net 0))
 (segment (start 17.387167 23.131201) (end 36.268382 23.131201) (width 5) (layer F.Cu) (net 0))
 (segment (start 36.268382 23.131201) (end 39.996 26.858819) (width 5) (layer F.Cu) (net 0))
 (segment (start 63.801 3.699) (end 63.801 9.479097) (width 5) (layer F.Cu) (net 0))
 (segment (start 63.801 9.479097) (end 61.885003 7.5631) (width 5) (layer F.Cu) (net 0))
 (segment (start 61.885003 7.5631) (end 39.996 7.5631) (width 5) (layer F.Cu) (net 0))
 (segment (start 39.996 7.5631) (end 39.996 11.354) (width 5) (layer F.Cu) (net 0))
 (segment (start 16.064 3.572) (end 16.064 8.223768) (width 5) (layer F.Cu) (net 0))
 (segment (start 16.064 8.223768) (end 17.387167 6.900601) (width 5) (layer F.Cu) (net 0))
 (segment (start 17.387167 6.900601) (end 36.268382 6.900601) (width 5) (layer F.Cu) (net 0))
 (segment (start 36.268382 6.900601) (end 39.996 10.628219) (width 5) (layer F.Cu) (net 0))
 (segment (start 39.996 10.628219) (end 39.996 11.354) (width 5) (layer F.Cu) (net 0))
 (segment (start 16.064 3.572) (end 39.948 3.572) (width 0.25) (layer F.Cu) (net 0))
 (segment (start 39.948 3.572) (end 39.996 3.62) (width 0.25) (layer F.Cu) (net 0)))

